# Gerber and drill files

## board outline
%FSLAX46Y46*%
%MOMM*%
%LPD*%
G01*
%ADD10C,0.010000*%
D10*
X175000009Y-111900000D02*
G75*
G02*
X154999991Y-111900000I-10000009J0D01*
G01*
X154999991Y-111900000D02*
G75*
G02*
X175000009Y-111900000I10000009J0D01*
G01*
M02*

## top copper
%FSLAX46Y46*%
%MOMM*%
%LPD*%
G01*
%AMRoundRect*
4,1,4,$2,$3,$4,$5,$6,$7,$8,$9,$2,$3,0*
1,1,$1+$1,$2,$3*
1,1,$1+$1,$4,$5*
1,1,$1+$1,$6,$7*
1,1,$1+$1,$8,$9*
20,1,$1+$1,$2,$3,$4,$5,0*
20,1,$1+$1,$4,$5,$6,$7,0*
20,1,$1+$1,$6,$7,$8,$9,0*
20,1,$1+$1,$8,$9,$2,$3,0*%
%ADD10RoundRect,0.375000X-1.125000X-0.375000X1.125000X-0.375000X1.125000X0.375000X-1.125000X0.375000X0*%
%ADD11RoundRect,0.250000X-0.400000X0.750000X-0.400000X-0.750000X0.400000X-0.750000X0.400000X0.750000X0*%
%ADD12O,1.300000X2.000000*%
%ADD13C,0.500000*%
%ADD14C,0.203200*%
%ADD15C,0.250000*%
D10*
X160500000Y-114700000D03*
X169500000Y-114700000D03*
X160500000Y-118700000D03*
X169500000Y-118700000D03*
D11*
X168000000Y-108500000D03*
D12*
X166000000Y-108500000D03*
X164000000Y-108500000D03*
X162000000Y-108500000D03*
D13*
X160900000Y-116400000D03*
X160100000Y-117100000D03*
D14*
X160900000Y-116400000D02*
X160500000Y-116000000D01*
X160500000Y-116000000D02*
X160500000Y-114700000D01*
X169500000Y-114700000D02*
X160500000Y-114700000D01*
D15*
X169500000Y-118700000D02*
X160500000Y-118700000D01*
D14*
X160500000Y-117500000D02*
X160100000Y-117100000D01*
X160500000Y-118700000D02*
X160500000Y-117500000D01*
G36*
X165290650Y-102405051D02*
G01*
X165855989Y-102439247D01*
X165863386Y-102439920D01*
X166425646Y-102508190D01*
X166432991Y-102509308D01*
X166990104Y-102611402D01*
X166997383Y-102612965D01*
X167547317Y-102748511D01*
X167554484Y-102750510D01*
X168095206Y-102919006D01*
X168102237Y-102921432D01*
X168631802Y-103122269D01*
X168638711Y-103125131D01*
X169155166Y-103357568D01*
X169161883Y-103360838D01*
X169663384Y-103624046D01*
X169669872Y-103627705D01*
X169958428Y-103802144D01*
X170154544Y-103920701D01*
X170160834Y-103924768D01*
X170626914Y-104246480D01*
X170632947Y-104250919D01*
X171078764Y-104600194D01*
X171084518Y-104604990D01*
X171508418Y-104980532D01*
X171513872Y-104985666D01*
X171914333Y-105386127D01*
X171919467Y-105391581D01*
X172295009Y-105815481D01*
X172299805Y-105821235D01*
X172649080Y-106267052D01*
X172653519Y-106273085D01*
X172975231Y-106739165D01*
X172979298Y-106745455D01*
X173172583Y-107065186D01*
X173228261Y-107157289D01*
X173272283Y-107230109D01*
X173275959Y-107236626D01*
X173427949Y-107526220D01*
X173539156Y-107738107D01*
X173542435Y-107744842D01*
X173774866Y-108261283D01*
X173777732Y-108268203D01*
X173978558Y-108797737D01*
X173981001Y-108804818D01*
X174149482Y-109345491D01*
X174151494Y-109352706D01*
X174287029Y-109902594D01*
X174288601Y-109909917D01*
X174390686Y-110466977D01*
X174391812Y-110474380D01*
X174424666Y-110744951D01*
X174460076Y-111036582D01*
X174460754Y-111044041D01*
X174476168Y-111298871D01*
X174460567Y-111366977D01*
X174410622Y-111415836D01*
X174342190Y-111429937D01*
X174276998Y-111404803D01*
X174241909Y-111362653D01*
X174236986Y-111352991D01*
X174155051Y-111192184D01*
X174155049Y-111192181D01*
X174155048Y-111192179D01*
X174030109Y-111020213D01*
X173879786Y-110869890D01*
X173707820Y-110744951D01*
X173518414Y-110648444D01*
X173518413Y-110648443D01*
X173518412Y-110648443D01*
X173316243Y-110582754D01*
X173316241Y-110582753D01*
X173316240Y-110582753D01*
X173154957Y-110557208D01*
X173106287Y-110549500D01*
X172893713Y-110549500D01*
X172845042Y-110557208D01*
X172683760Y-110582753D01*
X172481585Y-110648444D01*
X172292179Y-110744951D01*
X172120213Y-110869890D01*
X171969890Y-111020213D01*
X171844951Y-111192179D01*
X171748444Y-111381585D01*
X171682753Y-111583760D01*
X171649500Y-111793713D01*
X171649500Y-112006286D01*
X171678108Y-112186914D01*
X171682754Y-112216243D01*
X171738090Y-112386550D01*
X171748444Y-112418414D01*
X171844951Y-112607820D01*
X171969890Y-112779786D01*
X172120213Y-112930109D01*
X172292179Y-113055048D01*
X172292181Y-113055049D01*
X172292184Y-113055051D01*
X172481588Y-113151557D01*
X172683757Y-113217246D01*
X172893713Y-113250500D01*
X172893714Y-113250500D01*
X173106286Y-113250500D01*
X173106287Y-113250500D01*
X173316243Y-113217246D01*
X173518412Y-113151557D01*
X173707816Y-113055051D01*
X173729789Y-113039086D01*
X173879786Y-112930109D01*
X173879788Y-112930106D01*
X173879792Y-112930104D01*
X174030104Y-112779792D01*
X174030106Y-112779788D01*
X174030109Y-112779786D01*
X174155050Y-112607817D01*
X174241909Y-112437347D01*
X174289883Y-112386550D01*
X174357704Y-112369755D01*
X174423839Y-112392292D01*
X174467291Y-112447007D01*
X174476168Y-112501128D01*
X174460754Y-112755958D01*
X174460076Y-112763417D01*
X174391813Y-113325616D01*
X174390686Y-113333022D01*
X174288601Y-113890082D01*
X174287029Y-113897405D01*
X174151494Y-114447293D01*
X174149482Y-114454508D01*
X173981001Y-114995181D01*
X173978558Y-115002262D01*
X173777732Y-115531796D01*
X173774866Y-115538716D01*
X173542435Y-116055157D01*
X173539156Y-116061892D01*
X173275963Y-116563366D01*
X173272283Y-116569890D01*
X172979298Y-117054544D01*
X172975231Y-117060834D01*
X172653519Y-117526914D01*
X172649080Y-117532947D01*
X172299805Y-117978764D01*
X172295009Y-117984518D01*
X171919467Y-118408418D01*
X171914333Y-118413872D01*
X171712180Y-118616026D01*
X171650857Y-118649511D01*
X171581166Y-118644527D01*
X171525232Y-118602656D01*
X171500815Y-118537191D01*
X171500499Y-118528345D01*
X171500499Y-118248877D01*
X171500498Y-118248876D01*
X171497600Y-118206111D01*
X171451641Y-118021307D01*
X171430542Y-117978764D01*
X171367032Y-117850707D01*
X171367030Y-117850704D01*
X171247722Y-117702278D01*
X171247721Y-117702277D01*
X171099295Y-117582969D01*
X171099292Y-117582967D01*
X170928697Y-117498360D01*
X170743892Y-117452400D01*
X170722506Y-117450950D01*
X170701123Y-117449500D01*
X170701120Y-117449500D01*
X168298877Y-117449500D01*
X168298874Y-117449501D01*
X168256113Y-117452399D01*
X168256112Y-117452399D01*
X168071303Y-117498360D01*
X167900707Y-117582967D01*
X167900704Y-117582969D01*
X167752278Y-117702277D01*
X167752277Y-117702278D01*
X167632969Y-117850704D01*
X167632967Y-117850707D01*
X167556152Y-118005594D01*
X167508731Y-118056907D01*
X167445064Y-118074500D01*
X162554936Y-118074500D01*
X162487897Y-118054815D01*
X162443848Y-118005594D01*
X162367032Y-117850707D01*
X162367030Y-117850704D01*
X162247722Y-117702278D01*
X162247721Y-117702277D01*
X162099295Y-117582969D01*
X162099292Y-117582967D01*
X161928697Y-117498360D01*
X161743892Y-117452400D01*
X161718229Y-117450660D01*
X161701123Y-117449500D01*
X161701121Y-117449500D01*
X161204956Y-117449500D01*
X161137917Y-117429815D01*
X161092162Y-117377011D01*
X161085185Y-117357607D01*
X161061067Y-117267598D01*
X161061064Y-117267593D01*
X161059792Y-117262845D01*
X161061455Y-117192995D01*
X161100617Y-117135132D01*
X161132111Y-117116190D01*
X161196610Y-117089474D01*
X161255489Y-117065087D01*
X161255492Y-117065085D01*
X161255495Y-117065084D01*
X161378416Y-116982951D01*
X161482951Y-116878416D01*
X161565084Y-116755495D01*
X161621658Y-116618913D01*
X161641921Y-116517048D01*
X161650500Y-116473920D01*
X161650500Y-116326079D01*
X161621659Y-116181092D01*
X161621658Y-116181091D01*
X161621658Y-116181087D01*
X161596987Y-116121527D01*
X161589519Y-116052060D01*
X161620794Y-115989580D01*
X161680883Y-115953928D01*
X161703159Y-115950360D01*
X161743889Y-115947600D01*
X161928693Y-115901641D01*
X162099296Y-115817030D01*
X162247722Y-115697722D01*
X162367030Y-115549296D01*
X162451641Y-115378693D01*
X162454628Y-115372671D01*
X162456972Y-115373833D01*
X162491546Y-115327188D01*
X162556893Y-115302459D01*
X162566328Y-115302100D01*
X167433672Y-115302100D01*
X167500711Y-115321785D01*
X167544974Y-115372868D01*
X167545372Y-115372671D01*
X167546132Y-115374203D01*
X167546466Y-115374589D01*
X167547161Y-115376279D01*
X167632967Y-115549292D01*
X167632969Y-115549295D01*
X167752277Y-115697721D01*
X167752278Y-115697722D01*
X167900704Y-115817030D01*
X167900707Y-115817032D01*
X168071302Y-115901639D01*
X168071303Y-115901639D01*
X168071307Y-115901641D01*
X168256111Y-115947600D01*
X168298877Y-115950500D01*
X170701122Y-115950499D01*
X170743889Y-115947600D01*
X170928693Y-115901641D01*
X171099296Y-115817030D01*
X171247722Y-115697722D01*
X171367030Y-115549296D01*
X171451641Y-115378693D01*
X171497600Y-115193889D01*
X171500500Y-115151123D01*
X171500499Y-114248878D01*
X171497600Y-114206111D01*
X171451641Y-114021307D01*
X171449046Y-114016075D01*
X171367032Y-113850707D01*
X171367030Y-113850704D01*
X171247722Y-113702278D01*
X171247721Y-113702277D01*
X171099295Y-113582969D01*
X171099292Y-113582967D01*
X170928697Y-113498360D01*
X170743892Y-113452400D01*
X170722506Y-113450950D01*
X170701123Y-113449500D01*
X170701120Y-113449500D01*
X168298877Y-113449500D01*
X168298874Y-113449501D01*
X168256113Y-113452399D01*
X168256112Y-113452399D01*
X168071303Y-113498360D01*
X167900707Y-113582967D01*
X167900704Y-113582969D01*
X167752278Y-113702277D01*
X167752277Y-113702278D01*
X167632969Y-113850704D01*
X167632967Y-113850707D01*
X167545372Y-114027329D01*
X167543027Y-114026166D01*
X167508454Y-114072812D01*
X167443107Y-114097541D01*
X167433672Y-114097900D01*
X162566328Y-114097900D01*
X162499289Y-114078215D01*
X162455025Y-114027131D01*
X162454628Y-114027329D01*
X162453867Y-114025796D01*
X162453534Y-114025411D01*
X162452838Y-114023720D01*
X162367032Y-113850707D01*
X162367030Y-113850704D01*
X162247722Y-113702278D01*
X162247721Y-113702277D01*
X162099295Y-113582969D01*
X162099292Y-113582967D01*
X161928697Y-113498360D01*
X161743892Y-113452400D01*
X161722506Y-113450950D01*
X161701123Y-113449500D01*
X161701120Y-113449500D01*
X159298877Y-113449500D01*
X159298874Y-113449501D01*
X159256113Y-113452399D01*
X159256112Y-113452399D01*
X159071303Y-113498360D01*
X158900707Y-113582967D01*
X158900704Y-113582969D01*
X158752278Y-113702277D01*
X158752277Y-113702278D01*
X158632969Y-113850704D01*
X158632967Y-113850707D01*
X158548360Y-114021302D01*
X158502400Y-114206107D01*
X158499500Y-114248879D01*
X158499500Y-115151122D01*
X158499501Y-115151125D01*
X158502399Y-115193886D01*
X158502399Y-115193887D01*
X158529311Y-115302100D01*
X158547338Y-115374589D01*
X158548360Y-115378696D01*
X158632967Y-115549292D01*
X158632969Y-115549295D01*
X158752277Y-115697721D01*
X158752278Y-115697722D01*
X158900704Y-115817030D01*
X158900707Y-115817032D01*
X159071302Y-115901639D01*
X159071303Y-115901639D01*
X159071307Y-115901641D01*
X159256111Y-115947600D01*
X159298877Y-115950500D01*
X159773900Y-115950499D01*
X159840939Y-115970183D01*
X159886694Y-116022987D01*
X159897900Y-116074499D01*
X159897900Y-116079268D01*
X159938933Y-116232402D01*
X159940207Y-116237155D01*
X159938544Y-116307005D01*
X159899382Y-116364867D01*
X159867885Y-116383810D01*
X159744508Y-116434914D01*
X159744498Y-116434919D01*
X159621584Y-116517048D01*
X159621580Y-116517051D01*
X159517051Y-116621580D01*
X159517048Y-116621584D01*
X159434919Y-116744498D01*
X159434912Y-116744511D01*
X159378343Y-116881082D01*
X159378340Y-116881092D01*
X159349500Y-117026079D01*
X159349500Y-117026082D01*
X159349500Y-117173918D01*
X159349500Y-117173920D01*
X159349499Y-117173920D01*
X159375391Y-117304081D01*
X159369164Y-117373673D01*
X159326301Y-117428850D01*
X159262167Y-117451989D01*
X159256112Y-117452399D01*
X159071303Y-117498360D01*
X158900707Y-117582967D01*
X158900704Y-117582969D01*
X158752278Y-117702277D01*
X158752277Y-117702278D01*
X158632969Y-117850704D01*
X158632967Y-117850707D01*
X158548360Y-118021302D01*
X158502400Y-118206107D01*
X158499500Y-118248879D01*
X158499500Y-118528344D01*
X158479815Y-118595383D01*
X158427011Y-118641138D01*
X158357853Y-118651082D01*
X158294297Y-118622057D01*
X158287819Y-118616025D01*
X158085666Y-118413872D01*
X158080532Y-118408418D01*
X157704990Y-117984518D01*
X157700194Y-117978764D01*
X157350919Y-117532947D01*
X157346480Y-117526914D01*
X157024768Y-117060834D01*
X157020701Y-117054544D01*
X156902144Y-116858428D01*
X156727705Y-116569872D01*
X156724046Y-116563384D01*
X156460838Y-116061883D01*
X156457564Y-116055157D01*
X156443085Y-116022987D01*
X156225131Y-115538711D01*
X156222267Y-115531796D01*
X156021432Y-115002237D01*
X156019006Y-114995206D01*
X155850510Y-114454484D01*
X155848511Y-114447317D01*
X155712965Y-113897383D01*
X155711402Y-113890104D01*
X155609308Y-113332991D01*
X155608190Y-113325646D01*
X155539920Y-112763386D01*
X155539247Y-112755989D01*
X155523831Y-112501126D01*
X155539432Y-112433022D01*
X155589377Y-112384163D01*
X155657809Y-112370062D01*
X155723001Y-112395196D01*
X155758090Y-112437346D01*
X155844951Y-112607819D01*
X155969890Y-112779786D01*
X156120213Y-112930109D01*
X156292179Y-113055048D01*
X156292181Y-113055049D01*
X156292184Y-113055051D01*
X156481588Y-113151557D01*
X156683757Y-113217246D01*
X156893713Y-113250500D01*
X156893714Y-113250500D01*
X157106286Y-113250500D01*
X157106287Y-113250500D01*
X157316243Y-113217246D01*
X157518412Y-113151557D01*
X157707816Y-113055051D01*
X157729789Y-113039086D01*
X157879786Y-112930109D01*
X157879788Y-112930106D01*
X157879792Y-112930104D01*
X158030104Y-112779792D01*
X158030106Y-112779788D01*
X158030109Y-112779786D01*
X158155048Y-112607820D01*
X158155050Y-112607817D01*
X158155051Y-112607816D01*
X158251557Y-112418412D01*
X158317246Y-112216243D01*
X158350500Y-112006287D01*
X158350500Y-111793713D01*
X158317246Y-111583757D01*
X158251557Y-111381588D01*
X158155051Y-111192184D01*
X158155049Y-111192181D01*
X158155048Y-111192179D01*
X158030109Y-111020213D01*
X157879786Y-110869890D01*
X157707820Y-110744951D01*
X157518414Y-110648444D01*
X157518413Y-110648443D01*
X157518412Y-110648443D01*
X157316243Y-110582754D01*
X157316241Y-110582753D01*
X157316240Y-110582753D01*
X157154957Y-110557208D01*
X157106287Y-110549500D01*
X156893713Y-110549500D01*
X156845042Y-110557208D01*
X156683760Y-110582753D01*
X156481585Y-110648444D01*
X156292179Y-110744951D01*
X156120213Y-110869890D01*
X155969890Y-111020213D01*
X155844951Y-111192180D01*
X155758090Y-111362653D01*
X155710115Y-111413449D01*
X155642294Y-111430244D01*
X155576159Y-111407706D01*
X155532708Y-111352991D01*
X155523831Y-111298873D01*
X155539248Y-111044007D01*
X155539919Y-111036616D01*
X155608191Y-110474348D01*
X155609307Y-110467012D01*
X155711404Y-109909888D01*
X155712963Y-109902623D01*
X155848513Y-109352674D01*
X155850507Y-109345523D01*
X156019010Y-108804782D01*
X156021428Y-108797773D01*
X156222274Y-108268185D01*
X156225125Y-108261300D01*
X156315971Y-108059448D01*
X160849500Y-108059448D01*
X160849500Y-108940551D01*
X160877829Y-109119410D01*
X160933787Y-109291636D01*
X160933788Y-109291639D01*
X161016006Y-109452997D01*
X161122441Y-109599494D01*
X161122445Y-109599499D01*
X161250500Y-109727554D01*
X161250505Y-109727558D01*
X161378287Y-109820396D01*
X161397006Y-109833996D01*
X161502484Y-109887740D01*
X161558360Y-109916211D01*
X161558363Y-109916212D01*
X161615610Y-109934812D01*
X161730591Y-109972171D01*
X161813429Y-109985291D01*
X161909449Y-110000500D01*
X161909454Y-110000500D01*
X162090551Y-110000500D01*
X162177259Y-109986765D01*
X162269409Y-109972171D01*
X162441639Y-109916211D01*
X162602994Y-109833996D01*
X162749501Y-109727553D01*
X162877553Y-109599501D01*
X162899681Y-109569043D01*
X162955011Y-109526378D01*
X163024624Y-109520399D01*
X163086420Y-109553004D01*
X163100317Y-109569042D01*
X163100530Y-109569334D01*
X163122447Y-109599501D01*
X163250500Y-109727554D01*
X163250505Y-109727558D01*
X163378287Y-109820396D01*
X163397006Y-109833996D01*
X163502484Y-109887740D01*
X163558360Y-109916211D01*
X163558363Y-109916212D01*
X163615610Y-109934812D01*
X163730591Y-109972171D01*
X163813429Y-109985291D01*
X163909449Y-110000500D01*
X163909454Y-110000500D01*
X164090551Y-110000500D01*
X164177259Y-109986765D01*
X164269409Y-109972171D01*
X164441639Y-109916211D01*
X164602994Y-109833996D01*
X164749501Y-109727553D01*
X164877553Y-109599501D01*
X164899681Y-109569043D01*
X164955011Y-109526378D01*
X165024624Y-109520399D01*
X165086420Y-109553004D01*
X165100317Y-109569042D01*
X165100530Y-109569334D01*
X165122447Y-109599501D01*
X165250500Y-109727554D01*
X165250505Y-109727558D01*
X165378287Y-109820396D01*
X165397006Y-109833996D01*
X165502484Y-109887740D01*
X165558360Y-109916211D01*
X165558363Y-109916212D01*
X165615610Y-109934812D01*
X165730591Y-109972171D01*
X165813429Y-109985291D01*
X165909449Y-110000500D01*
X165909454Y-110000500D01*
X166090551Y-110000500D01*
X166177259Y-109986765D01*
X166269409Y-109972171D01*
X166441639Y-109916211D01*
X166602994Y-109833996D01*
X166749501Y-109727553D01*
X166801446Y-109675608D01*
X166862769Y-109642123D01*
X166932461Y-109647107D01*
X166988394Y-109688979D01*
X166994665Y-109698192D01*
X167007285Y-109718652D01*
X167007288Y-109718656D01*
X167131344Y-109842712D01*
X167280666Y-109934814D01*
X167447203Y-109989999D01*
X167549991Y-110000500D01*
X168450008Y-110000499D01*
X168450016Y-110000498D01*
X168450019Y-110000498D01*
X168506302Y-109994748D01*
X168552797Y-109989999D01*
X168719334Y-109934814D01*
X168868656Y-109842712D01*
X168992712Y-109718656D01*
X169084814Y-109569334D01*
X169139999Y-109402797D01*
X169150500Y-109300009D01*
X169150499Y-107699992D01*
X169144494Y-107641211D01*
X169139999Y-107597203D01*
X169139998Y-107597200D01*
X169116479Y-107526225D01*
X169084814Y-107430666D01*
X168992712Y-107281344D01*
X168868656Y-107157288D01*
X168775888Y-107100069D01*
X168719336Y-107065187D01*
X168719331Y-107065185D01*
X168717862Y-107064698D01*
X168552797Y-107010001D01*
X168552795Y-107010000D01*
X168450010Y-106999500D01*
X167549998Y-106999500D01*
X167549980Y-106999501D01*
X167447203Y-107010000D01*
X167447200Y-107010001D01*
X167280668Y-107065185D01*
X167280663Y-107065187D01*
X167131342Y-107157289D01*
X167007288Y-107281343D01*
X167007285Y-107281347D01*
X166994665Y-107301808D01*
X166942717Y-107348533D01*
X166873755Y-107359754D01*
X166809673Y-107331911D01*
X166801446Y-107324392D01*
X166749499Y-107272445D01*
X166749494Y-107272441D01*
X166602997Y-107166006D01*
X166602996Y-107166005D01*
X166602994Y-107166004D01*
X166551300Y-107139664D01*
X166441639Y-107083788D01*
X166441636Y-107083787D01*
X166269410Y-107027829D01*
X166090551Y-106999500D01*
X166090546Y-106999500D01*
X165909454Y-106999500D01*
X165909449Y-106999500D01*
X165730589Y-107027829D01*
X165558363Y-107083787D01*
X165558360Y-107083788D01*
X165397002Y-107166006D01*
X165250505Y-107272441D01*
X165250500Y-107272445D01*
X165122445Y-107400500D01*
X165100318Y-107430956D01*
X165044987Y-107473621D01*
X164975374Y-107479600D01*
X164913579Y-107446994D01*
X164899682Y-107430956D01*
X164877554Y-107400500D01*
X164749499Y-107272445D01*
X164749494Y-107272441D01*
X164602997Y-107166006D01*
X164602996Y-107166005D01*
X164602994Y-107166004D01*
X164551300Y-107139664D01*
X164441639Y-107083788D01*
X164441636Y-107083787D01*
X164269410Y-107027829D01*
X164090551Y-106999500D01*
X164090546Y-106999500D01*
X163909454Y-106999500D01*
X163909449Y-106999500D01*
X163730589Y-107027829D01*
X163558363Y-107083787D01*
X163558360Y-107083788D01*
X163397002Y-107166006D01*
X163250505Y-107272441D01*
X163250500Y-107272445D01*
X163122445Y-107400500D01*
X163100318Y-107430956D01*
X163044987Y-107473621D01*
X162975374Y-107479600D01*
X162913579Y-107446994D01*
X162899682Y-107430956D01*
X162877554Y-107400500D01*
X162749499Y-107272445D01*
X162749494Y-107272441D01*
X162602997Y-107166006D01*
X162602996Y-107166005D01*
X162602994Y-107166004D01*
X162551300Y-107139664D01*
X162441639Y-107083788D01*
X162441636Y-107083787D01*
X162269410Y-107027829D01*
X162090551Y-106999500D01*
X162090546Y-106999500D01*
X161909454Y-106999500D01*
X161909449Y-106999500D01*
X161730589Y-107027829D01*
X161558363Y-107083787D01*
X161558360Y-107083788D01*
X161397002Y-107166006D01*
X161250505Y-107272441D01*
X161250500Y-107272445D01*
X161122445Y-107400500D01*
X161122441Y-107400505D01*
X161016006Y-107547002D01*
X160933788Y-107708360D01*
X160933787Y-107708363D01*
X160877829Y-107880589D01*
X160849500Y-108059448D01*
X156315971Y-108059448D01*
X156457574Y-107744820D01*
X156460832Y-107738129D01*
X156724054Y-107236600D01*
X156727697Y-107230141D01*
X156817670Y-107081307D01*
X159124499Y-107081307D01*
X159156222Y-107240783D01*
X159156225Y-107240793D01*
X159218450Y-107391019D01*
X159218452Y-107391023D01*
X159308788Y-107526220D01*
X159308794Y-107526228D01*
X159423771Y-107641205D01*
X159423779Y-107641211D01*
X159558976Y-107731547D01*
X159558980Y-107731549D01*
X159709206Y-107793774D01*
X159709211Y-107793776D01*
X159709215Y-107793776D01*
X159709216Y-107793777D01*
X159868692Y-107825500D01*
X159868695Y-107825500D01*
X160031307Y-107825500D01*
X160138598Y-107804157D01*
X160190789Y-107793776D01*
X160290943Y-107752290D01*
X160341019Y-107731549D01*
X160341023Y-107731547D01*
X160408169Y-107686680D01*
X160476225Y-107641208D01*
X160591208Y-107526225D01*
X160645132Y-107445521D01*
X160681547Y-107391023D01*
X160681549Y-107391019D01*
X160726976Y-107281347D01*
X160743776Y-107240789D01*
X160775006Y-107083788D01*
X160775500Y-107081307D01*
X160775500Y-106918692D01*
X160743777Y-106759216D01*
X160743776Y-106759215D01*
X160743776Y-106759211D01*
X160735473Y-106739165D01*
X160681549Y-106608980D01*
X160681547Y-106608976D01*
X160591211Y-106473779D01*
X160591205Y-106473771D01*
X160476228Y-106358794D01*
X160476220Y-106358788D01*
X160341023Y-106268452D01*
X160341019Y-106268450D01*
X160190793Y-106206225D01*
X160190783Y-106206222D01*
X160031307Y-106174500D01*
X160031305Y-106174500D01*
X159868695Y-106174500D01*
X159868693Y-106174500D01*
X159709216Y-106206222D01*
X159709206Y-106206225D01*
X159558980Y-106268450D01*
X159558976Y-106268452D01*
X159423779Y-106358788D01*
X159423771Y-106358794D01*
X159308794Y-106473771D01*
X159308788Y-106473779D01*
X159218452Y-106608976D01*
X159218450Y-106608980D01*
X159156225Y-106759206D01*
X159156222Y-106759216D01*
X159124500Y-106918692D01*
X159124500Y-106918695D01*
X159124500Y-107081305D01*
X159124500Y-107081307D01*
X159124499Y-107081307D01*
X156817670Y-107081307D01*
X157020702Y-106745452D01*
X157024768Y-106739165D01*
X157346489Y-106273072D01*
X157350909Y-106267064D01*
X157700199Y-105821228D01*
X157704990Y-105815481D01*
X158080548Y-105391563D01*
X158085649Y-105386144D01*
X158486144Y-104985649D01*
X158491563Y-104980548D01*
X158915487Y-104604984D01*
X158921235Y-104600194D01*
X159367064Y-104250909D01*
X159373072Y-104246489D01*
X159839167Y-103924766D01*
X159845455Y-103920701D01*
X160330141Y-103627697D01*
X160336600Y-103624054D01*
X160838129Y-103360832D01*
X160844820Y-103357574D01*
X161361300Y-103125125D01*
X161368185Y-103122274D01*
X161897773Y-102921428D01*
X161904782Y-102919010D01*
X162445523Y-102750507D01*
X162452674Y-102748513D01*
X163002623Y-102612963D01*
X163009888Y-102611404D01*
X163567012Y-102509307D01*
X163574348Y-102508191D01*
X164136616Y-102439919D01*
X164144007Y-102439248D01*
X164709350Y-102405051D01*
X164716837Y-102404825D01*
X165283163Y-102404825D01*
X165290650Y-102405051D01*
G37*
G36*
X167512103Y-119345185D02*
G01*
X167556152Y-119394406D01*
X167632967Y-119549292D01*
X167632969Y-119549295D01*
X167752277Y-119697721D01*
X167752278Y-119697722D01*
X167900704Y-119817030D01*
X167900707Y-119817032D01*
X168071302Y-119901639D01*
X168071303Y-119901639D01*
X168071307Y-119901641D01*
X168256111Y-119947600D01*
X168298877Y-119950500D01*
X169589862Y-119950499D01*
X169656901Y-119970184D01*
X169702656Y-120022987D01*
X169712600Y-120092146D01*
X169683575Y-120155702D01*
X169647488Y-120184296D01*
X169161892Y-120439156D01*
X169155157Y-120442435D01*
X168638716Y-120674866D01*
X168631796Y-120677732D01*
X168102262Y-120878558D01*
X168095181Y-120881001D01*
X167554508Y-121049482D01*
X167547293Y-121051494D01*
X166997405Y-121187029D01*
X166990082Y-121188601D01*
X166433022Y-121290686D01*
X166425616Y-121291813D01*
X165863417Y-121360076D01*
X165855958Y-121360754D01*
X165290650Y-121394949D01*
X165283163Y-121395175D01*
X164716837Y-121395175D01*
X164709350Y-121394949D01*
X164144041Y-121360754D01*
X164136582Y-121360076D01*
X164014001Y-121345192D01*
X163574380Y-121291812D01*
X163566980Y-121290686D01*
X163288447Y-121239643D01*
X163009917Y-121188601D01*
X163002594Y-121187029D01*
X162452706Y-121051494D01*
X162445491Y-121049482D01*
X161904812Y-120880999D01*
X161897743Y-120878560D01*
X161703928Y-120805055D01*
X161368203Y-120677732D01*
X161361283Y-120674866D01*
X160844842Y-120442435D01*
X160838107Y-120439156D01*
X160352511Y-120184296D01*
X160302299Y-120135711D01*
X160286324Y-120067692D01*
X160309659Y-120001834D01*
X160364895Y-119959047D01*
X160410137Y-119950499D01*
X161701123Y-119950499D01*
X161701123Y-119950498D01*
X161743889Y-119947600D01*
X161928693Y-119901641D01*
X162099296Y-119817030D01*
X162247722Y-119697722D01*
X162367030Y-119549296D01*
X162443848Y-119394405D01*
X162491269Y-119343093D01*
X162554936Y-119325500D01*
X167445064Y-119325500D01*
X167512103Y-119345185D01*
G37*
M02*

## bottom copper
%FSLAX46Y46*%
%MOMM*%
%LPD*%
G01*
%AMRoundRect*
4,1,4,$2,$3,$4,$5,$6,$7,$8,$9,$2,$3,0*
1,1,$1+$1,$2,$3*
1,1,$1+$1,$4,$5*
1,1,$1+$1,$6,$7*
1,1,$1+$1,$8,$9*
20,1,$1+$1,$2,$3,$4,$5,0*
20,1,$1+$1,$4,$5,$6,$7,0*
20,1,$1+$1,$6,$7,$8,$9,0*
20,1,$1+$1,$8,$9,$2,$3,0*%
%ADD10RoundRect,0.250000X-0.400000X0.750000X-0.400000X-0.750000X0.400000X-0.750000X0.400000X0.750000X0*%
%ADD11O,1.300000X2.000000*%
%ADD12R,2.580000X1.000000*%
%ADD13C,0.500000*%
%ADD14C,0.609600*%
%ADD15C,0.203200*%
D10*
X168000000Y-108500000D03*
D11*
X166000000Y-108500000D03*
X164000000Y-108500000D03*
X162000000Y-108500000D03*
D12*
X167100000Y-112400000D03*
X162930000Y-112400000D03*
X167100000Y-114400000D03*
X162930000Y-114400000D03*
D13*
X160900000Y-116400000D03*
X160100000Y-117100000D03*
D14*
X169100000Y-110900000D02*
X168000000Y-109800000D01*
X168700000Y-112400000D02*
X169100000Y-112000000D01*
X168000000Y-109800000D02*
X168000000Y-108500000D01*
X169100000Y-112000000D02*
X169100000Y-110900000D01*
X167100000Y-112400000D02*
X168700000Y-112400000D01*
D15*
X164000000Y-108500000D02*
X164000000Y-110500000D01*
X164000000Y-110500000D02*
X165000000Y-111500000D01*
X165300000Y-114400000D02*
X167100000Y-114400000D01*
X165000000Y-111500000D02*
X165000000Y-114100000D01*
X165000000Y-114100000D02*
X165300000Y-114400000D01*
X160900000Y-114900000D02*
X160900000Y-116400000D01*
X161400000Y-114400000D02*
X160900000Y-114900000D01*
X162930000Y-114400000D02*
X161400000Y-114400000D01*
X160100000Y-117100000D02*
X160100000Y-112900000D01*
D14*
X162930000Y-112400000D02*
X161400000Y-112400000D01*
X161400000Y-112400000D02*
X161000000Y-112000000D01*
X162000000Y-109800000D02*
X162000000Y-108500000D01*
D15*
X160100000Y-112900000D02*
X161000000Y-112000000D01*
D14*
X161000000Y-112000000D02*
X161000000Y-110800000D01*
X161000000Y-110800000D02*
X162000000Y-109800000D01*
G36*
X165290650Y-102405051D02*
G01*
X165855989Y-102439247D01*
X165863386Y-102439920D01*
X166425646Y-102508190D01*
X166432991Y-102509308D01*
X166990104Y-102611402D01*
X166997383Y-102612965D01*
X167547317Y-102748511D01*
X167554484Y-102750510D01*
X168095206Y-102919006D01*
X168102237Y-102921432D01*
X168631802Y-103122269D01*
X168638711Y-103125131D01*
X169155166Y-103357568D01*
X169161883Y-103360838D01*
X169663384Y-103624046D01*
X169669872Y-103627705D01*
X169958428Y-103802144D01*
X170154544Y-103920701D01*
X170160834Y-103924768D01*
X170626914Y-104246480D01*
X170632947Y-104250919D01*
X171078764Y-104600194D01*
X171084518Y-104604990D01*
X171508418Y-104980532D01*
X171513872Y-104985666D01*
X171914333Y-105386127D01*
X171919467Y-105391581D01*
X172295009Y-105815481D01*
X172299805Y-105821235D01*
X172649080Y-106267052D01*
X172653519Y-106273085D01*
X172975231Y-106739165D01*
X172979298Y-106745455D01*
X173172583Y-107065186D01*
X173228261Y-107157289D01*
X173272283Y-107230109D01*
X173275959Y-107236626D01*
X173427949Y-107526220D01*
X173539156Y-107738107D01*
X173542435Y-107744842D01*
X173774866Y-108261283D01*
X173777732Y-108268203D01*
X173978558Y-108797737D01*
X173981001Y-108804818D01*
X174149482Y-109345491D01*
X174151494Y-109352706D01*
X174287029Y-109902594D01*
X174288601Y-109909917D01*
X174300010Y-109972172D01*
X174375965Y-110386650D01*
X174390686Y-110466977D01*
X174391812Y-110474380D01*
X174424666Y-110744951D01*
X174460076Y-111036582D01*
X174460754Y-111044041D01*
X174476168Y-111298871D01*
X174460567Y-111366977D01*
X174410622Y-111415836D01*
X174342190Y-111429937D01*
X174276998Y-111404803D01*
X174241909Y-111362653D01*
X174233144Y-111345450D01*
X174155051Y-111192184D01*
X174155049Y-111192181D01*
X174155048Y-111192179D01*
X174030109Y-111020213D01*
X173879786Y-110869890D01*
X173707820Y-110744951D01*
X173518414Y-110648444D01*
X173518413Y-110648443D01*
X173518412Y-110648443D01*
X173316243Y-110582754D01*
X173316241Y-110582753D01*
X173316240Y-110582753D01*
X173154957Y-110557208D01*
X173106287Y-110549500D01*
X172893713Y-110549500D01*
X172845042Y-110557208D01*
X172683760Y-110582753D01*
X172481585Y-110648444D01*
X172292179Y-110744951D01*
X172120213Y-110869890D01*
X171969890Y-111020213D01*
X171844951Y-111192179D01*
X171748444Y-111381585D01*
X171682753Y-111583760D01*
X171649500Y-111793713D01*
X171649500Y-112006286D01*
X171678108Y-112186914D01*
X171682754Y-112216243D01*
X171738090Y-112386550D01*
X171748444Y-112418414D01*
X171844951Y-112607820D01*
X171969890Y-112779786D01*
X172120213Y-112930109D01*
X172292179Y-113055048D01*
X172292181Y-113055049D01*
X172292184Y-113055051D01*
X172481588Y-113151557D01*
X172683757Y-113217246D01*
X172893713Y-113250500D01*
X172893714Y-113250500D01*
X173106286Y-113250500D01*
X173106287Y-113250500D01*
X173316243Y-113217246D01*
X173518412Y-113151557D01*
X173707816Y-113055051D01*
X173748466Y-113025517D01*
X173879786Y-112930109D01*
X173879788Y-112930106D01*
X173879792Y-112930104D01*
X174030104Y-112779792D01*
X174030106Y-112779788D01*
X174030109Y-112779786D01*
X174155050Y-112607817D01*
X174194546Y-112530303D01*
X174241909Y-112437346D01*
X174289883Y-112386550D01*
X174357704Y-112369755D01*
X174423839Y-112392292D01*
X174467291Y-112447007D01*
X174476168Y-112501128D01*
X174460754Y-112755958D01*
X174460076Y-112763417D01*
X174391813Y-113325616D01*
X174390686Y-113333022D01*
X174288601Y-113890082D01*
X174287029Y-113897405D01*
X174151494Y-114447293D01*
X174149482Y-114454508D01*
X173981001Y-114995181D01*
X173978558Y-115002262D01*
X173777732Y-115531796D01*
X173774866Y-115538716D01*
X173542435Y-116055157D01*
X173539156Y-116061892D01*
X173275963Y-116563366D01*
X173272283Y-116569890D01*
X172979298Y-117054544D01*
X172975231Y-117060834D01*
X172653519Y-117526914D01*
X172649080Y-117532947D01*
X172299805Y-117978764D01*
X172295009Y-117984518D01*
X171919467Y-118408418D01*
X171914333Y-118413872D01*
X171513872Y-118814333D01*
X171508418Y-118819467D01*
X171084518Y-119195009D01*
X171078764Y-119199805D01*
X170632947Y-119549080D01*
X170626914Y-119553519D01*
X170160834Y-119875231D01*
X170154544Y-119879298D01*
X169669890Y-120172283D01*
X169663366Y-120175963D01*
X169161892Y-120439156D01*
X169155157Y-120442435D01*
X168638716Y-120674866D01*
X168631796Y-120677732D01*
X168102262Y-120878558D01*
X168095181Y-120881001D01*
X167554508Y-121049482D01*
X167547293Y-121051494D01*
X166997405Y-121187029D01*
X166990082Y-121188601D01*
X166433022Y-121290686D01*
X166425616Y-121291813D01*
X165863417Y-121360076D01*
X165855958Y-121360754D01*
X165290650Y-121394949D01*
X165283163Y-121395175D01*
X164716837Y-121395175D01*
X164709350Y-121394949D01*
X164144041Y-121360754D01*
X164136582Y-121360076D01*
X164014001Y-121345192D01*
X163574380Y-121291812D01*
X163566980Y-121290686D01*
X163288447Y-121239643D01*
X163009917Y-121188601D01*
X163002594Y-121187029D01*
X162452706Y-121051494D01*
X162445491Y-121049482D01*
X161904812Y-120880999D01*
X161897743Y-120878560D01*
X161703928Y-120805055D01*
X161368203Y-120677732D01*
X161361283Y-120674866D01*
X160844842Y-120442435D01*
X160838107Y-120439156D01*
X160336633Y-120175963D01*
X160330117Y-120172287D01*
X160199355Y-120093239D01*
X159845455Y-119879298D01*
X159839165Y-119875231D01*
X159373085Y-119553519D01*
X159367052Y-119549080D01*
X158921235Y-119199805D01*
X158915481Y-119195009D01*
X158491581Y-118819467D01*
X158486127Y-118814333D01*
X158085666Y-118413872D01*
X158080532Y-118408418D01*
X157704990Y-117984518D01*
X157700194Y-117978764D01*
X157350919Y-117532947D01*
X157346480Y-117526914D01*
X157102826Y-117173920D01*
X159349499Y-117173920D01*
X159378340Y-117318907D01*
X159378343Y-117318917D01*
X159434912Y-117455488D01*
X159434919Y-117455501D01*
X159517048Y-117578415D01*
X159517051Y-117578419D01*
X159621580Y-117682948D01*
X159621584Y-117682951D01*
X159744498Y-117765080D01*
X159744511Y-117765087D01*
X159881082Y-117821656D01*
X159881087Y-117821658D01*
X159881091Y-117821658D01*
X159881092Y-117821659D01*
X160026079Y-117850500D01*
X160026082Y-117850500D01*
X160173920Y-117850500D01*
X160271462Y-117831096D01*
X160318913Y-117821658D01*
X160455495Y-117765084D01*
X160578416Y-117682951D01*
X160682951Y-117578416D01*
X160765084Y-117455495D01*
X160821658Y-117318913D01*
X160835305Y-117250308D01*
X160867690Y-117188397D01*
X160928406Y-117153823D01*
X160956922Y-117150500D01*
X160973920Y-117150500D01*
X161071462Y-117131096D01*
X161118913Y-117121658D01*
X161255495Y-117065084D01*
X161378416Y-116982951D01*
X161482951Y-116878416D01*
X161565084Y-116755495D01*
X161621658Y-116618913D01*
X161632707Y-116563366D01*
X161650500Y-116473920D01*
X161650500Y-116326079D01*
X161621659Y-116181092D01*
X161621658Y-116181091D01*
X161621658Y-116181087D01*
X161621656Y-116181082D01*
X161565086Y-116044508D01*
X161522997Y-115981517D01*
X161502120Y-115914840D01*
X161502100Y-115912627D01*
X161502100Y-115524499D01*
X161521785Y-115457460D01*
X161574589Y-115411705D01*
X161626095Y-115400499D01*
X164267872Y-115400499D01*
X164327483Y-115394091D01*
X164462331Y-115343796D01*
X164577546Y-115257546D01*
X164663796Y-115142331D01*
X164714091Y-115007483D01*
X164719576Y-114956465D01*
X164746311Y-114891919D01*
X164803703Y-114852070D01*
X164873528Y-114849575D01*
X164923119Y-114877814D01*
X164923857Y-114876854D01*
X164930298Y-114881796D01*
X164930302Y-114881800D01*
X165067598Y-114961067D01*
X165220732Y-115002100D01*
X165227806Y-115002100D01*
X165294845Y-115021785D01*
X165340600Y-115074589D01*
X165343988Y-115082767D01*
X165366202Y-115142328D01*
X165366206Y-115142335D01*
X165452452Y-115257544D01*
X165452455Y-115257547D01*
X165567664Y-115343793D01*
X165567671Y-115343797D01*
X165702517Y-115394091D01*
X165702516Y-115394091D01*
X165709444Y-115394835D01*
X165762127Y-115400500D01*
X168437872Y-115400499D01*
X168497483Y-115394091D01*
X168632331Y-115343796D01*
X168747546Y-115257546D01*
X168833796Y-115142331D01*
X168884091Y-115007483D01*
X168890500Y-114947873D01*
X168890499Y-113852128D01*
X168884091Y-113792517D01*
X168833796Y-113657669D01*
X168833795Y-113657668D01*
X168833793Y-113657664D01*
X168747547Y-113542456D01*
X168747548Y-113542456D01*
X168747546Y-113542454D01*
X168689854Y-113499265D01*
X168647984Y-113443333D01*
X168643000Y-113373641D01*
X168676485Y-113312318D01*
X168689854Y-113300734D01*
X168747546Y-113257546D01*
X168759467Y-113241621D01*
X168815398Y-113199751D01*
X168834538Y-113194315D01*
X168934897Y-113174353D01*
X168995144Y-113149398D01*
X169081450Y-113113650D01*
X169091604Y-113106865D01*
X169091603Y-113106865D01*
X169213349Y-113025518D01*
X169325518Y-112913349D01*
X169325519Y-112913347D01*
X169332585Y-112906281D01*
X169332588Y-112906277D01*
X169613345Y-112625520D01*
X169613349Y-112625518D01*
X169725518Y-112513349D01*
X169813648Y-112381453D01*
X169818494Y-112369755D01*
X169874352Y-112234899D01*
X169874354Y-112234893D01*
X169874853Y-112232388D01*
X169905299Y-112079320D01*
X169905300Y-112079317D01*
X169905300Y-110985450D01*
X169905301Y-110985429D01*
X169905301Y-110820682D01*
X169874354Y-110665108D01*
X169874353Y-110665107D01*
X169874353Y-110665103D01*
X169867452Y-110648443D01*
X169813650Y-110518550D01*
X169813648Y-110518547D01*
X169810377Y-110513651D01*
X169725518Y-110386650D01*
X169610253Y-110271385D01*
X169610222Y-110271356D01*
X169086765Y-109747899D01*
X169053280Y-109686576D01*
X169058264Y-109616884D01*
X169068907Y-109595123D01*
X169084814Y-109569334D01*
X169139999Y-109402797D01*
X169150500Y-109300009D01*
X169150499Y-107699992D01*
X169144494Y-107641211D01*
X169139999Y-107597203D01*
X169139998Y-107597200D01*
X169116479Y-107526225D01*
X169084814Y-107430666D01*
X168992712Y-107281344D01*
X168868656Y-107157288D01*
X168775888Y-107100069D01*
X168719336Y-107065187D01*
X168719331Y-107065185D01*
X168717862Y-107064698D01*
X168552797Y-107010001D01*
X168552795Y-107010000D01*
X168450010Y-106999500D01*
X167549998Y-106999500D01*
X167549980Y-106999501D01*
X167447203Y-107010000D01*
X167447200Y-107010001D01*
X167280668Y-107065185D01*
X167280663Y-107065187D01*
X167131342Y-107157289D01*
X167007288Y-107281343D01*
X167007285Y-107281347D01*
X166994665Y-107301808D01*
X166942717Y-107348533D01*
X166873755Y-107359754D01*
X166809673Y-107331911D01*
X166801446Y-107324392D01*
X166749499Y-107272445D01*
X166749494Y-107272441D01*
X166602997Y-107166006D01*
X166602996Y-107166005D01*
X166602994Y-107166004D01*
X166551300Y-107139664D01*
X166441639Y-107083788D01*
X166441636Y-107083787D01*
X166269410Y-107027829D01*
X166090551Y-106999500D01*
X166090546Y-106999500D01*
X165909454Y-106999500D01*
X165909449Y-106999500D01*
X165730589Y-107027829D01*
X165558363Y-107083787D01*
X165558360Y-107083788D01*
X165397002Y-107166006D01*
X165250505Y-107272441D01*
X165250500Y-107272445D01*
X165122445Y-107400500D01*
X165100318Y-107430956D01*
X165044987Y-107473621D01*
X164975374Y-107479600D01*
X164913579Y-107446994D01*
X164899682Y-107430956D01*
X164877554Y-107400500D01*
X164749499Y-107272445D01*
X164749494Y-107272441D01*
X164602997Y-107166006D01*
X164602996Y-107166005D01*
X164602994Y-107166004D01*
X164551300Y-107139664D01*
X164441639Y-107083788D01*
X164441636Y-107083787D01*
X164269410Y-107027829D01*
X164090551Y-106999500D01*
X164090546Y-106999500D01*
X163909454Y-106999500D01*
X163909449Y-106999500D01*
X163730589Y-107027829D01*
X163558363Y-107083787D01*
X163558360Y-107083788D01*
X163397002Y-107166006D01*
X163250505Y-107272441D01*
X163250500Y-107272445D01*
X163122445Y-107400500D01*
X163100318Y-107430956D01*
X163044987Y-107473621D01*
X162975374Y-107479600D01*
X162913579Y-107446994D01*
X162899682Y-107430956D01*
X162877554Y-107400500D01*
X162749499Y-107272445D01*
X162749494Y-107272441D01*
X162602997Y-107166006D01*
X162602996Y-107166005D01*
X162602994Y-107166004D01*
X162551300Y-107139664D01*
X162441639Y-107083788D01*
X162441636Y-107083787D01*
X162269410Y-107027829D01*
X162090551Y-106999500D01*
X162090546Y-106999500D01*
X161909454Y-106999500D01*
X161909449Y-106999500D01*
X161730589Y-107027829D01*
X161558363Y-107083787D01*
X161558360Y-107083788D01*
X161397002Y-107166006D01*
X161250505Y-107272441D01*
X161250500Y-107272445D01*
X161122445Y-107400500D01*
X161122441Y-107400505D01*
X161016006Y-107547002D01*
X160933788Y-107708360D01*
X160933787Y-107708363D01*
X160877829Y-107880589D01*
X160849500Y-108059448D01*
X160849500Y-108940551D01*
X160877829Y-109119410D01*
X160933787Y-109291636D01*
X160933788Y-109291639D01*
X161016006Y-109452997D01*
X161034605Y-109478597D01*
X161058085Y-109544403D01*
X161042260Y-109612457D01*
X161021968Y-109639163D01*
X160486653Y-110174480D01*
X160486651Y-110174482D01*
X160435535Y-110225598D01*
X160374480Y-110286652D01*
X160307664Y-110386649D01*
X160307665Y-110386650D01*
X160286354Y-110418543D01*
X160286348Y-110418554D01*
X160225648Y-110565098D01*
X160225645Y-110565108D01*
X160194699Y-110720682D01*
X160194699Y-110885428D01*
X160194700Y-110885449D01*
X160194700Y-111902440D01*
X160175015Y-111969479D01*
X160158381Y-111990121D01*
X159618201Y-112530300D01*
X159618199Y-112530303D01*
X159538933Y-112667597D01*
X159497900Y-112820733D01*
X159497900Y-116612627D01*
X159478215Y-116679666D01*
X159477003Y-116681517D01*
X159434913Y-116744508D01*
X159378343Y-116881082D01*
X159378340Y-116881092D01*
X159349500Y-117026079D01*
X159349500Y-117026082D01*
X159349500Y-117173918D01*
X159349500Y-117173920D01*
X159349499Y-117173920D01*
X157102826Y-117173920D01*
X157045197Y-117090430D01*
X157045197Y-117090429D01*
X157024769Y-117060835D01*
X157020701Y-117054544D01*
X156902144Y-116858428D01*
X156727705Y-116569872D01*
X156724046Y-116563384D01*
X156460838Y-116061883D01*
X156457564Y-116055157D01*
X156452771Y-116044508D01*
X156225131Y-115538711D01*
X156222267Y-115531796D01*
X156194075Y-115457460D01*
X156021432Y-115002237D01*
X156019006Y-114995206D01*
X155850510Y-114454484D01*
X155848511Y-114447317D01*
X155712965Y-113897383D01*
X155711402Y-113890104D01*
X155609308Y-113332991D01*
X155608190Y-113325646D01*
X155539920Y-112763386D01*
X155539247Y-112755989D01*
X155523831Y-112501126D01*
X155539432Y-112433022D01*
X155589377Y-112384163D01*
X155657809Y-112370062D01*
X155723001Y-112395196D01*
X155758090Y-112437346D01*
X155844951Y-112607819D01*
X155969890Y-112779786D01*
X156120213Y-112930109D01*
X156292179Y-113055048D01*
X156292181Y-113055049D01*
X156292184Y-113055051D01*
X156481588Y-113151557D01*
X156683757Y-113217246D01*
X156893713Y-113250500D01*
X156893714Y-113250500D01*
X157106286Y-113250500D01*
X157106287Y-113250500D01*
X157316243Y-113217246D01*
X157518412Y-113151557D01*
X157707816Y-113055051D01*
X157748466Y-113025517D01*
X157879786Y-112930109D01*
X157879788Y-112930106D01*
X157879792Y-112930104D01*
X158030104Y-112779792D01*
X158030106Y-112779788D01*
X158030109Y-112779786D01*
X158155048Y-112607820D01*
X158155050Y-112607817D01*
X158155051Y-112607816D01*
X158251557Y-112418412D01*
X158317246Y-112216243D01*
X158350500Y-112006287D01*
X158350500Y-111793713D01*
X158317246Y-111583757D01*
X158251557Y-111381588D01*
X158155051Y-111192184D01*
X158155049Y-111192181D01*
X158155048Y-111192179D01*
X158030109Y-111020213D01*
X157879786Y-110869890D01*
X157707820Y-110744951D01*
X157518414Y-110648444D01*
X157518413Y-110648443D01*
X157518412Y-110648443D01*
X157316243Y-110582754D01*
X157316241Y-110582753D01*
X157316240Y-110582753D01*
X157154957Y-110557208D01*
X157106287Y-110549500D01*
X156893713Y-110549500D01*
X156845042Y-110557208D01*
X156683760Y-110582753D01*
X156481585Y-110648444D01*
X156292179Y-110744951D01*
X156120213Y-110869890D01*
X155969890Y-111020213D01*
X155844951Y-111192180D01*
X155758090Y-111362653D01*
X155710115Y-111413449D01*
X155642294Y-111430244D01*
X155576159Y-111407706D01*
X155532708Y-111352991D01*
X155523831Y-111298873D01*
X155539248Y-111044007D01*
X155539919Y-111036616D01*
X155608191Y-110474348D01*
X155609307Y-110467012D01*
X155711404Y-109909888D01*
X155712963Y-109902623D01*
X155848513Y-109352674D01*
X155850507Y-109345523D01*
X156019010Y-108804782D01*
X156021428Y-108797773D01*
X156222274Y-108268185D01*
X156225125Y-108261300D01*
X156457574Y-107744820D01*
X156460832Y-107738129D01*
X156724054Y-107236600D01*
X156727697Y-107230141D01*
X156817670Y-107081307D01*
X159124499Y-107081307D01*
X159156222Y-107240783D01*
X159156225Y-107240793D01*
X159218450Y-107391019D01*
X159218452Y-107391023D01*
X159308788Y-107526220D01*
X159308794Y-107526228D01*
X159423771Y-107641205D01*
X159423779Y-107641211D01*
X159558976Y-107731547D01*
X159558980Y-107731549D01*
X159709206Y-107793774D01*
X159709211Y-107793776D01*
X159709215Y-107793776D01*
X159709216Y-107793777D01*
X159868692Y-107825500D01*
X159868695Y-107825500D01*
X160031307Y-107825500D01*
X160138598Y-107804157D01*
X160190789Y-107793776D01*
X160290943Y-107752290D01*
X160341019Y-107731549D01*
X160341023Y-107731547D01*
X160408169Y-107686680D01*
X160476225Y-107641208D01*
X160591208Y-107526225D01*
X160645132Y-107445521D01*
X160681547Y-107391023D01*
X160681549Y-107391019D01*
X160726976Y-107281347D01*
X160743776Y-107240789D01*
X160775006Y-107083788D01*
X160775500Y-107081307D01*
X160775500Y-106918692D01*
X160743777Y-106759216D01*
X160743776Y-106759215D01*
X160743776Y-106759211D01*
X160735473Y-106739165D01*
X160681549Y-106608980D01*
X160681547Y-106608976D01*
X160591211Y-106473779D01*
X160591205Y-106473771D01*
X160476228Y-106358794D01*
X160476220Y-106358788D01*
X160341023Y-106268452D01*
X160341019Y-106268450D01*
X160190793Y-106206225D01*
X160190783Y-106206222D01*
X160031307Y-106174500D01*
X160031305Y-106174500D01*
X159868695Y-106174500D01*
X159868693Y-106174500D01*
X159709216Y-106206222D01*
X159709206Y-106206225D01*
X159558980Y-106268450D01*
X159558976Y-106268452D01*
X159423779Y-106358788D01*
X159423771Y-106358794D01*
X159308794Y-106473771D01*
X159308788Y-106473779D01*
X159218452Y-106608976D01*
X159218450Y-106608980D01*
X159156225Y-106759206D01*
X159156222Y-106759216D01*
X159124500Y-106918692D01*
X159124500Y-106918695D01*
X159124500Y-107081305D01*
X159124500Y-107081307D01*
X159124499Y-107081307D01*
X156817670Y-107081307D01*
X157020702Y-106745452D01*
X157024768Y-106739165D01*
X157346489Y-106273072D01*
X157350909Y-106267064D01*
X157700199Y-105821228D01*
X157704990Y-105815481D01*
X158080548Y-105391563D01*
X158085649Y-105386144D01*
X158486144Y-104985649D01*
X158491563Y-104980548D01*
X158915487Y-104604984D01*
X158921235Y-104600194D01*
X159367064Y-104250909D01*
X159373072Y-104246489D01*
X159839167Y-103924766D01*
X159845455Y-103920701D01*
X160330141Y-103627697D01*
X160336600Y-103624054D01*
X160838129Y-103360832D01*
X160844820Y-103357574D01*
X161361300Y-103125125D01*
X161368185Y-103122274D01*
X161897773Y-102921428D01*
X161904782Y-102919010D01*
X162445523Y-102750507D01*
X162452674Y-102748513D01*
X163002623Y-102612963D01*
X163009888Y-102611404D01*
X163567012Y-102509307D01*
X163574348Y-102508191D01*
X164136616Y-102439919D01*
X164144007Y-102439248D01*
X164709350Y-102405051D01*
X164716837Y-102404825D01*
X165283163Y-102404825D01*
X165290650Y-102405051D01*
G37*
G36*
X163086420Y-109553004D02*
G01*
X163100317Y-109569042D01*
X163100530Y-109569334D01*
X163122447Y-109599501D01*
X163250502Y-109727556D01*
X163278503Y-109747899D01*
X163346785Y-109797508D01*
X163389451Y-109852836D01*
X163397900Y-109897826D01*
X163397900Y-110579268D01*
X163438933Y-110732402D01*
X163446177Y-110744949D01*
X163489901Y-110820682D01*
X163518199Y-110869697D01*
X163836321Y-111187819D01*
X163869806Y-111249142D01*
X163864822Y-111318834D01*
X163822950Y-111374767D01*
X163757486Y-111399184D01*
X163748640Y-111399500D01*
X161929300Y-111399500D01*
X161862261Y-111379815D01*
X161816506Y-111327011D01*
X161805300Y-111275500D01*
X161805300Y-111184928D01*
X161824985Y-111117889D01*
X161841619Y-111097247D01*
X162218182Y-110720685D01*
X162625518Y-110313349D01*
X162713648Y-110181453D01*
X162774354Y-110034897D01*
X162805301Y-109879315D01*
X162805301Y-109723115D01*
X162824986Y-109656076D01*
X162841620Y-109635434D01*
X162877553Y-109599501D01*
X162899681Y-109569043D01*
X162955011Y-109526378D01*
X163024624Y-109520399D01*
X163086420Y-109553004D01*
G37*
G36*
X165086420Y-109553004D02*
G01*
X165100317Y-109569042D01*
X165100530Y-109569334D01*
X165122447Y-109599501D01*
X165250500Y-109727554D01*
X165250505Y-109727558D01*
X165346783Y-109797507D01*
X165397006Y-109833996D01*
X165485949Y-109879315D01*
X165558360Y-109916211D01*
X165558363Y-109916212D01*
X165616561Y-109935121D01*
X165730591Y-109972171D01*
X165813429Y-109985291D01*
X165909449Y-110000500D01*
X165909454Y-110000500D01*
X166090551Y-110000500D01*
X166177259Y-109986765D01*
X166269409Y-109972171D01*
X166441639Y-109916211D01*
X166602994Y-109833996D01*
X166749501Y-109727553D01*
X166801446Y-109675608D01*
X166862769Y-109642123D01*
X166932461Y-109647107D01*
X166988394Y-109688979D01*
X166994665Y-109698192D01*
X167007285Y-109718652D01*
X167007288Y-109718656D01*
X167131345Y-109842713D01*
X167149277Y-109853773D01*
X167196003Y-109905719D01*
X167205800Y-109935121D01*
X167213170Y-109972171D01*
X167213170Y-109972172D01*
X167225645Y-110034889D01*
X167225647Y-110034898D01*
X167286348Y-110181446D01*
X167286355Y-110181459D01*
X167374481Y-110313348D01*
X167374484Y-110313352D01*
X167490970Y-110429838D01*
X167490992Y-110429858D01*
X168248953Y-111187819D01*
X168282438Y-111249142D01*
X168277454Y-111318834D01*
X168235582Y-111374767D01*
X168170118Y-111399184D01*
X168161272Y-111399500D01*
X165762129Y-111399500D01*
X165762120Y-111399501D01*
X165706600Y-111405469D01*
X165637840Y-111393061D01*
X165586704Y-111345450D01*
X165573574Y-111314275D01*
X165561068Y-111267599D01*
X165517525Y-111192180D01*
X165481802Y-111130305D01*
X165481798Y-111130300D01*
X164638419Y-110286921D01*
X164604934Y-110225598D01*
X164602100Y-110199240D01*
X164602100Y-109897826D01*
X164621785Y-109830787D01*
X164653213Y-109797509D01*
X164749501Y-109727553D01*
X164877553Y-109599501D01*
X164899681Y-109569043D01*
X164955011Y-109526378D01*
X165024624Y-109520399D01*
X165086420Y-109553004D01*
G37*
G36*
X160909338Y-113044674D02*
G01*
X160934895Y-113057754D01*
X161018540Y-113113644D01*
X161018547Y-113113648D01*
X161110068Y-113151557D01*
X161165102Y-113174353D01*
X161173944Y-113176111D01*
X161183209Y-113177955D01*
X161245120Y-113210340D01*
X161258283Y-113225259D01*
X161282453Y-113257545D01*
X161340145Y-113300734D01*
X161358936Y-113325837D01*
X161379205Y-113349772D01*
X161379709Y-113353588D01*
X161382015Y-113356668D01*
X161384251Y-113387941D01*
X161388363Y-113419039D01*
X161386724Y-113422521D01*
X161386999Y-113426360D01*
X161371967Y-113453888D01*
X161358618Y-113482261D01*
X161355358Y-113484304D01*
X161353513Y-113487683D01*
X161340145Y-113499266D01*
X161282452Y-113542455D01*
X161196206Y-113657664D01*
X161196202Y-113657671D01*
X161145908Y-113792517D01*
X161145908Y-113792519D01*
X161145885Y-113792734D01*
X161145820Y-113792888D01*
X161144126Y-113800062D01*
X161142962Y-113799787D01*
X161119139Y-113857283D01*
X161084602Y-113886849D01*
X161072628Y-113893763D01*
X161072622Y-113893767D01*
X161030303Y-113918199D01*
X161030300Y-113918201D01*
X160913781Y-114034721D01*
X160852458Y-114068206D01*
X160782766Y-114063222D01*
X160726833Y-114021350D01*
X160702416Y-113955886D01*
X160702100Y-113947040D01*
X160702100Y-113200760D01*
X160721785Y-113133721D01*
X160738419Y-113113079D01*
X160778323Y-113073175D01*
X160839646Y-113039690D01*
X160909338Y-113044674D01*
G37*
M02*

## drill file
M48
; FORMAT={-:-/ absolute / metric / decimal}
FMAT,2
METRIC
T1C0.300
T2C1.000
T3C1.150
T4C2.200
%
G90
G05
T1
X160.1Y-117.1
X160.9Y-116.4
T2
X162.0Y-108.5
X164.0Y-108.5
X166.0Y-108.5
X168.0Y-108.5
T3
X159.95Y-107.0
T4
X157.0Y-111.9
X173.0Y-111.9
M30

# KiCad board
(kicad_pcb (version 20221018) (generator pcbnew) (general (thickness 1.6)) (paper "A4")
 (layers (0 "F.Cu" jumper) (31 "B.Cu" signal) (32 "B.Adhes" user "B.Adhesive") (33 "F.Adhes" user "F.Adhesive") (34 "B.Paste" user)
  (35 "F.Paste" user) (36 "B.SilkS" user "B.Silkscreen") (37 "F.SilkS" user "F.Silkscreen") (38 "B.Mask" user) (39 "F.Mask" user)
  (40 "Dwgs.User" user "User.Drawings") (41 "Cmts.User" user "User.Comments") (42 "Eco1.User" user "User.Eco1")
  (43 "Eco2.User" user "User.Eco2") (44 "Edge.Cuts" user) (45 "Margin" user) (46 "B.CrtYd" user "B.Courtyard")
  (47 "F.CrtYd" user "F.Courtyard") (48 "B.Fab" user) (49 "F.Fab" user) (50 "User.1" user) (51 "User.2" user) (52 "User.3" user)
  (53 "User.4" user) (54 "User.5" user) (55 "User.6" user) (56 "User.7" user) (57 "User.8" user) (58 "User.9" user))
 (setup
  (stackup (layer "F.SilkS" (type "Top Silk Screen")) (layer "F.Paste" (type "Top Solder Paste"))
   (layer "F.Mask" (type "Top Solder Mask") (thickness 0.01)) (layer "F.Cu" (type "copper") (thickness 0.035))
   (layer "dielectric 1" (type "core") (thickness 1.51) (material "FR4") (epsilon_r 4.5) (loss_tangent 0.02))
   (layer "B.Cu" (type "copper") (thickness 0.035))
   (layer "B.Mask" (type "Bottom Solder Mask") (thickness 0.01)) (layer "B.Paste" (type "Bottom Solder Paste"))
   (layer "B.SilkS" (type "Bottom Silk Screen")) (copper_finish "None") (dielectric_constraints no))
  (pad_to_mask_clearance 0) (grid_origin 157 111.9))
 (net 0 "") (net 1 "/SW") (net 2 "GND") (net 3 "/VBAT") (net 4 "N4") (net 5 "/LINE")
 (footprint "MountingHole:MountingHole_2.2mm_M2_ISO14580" (layer "F.Cu") (at 157 111.9)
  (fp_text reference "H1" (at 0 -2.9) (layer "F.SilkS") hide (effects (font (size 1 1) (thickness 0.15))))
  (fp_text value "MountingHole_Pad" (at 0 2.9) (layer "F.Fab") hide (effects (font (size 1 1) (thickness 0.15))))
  (pad "" np_thru_hole circle (at 0 0) (size 2.2 2.2) (drill 2.2) (layers "*.Cu" "*.Mask")))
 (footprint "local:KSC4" (layer "F.Cu") (at 165 116.7)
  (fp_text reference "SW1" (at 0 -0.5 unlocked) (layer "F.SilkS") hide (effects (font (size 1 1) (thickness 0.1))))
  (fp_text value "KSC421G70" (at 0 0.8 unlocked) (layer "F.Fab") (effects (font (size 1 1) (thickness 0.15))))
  (pad "1" smd roundrect (at -4.5 -2) (size 3 1.5) (layers "F.Cu" "F.Paste" "F.Mask") (roundrect_rratio 0.25) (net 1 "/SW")
   (thermal_bridge_angle 45))
  (pad "2" smd roundrect (at 4.5 -2) (size 3 1.5) (layers "F.Cu" "F.Paste" "F.Mask") (roundrect_rratio 0.25) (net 1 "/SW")
   (thermal_bridge_angle 45))
  (pad "3" smd roundrect (at -4.5 2) (size 3 1.5) (layers "F.Cu" "F.Paste" "F.Mask") (roundrect_rratio 0.25) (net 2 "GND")
   (thermal_bridge_angle 45))
  (pad "4" smd roundrect (at 4.5 2) (size 3 1.5) (layers "F.Cu" "F.Paste" "F.Mask") (roundrect_rratio 0.25) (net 2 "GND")
   (thermal_bridge_angle 45)))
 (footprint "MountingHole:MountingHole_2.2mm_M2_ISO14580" (layer "F.Cu") (at 173 111.9)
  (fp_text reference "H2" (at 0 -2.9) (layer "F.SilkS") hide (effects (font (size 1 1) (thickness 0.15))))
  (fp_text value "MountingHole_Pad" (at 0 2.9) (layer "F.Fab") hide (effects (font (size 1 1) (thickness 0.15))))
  (pad "" np_thru_hole circle (at 0 0) (size 2.2 2.2) (drill 2.2) (layers "*.Cu" "*.Mask")))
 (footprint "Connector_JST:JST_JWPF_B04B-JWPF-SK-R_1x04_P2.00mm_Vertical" (layer "F.Cu") (at 168 108.5 -90)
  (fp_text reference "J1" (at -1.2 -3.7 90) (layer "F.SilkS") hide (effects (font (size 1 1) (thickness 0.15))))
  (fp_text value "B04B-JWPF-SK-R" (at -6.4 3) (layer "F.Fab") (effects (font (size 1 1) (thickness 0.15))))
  (pad "" np_thru_hole circle (at -1.5 8.05 270) (size 1.15 1.15) (drill 1.15) (layers "*.Cu" "*.Mask"))
  (pad "1" thru_hole roundrect (at 0 0 270) (size 2 1.3) (drill 1) (layers "*.Cu" "*.Mask") (roundrect_rratio 0.1923076923) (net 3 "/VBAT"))
  (pad "2" thru_hole oval (at 0 2 270) (size 2 1.3) (drill 1) (layers "*.Cu" "*.Mask") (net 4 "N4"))
  (pad "3" thru_hole oval (at 0 4 270) (size 2 1.3) (drill 1) (layers "*.Cu" "*.Mask") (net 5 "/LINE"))
  (pad "4" thru_hole oval (at 0 6 270) (size 2 1.3) (drill 1) (layers "*.Cu" "*.Mask") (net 2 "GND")))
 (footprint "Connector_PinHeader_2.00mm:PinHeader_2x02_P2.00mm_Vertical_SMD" (layer "B.Cu") (at 165.015 113.4 180)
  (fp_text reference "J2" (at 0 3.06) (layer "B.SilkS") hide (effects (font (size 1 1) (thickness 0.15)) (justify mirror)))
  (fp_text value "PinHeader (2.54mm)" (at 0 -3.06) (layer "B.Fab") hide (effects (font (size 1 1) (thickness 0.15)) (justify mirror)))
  (pad "1" smd rect (at -2.085 1 180) (size 2.58 1) (layers "B.Cu" "B.Paste" "B.Mask") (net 3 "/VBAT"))
  (pad "2" smd rect (at 2.085 1 180) (size 2.58 1) (layers "B.Cu" "B.Paste" "B.Mask") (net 2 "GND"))
  (pad "3" smd rect (at -2.085 -1 180) (size 2.58 1) (layers "B.Cu" "B.Paste" "B.Mask") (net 5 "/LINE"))
  (pad "4" smd rect (at 2.085 -1 180) (size 2.58 1) (layers "B.Cu" "B.Paste" "B.Mask") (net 1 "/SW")))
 (gr_circle (center 165 111.9) (end 175.000009 111.9) (stroke (width 0.01) (type solid)) (fill none) (layer "Edge.Cuts"))
 (segment (start 169.1 110.9) (end 168 109.8) (width 0.6096) (layer "B.Cu") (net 3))
 (segment (start 168.7 112.4) (end 169.1 112) (width 0.6096) (layer "B.Cu") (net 3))
 (segment (start 168 109.8) (end 168 108.5) (width 0.6096) (layer "B.Cu") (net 3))
 (segment (start 169.1 112) (end 169.1 110.9) (width 0.6096) (layer "B.Cu") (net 3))
 (segment (start 167.1 112.4) (end 168.7 112.4) (width 0.6096) (layer "B.Cu") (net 3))
 (segment (start 164 108.5) (end 164 110.5) (width 0.2032) (layer "B.Cu") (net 5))
 (segment (start 164 110.5) (end 165 111.5) (width 0.2032) (layer "B.Cu") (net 5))
 (segment (start 165.3 114.4) (end 167.1 114.4) (width 0.2032) (layer "B.Cu") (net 5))
 (segment (start 165 111.5) (end 165 114.1) (width 0.2032) (layer "B.Cu") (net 5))
 (segment (start 165 114.1) (end 165.3 114.4) (width 0.2032) (layer "B.Cu") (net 5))
 (segment (start 160.9 116.4) (end 160.5 116) (width 0.2032) (layer "F.Cu") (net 1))
 (segment (start 160.5 116) (end 160.5 114.7) (width 0.2032) (layer "F.Cu") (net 1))
 (segment (start 169.5 114.7) (end 160.5 114.7) (width 0.2032) (layer "F.Cu") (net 1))
 (via (at 160.9 116.4) (size 0.5) (drill 0.3) (layers "F.Cu" "B.Cu") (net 1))
 (segment (start 160.9 114.9) (end 160.9 116.4) (width 0.2032) (layer "B.Cu") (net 1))
 (segment (start 161.4 114.4) (end 160.9 114.9) (width 0.2032) (layer "B.Cu") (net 1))
 (segment (start 162.93 114.4) (end 161.4 114.4) (width 0.2032) (layer "B.Cu") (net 1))
 (segment (start 169.5 118.7) (end 160.5 118.7) (width 0.25) (layer "F.Cu") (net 2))
 (segment (start 160.5 117.5) (end 160.1 117.1) (width 0.2032) (layer "F.Cu") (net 2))
 (segment (start 160.5 118.7) (end 160.5 117.5) (width 0.2032) (layer "F.Cu") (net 2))
 (via (at 160.1 117.1) (size 0.5) (drill 0.3) (layers "F.Cu" "B.Cu") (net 2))
 (segment (start 160.1 117.1) (end 160.1 112.9) (width 0.2032) (layer "B.Cu") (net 2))
 (segment (start 162.93 112.4) (end 161.4 112.4) (width 0.6096) (layer "B.Cu") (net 2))
 (segment (start 161.4 112.4) (end 161 112) (width 0.6096) (layer "B.Cu") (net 2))
 (segment (start 162 109.8) (end 162 108.5) (width 0.6096) (layer "B.Cu") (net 2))
 (segment (start 160.1 112.9) (end 161 112) (width 0.2032) (layer "B.Cu") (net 2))
 (segment (start 161 112) (end 161 110.8) (width 0.6096) (layer "B.Cu") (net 2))
 (segment (start 161 110.8) (end 162 109.8) (width 0.6096) (layer "B.Cu") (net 2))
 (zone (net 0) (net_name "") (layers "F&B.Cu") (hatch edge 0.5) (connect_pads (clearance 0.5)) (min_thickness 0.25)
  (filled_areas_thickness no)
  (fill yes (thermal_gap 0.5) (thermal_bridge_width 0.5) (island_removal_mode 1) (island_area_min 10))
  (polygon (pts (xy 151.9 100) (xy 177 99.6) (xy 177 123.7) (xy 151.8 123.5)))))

